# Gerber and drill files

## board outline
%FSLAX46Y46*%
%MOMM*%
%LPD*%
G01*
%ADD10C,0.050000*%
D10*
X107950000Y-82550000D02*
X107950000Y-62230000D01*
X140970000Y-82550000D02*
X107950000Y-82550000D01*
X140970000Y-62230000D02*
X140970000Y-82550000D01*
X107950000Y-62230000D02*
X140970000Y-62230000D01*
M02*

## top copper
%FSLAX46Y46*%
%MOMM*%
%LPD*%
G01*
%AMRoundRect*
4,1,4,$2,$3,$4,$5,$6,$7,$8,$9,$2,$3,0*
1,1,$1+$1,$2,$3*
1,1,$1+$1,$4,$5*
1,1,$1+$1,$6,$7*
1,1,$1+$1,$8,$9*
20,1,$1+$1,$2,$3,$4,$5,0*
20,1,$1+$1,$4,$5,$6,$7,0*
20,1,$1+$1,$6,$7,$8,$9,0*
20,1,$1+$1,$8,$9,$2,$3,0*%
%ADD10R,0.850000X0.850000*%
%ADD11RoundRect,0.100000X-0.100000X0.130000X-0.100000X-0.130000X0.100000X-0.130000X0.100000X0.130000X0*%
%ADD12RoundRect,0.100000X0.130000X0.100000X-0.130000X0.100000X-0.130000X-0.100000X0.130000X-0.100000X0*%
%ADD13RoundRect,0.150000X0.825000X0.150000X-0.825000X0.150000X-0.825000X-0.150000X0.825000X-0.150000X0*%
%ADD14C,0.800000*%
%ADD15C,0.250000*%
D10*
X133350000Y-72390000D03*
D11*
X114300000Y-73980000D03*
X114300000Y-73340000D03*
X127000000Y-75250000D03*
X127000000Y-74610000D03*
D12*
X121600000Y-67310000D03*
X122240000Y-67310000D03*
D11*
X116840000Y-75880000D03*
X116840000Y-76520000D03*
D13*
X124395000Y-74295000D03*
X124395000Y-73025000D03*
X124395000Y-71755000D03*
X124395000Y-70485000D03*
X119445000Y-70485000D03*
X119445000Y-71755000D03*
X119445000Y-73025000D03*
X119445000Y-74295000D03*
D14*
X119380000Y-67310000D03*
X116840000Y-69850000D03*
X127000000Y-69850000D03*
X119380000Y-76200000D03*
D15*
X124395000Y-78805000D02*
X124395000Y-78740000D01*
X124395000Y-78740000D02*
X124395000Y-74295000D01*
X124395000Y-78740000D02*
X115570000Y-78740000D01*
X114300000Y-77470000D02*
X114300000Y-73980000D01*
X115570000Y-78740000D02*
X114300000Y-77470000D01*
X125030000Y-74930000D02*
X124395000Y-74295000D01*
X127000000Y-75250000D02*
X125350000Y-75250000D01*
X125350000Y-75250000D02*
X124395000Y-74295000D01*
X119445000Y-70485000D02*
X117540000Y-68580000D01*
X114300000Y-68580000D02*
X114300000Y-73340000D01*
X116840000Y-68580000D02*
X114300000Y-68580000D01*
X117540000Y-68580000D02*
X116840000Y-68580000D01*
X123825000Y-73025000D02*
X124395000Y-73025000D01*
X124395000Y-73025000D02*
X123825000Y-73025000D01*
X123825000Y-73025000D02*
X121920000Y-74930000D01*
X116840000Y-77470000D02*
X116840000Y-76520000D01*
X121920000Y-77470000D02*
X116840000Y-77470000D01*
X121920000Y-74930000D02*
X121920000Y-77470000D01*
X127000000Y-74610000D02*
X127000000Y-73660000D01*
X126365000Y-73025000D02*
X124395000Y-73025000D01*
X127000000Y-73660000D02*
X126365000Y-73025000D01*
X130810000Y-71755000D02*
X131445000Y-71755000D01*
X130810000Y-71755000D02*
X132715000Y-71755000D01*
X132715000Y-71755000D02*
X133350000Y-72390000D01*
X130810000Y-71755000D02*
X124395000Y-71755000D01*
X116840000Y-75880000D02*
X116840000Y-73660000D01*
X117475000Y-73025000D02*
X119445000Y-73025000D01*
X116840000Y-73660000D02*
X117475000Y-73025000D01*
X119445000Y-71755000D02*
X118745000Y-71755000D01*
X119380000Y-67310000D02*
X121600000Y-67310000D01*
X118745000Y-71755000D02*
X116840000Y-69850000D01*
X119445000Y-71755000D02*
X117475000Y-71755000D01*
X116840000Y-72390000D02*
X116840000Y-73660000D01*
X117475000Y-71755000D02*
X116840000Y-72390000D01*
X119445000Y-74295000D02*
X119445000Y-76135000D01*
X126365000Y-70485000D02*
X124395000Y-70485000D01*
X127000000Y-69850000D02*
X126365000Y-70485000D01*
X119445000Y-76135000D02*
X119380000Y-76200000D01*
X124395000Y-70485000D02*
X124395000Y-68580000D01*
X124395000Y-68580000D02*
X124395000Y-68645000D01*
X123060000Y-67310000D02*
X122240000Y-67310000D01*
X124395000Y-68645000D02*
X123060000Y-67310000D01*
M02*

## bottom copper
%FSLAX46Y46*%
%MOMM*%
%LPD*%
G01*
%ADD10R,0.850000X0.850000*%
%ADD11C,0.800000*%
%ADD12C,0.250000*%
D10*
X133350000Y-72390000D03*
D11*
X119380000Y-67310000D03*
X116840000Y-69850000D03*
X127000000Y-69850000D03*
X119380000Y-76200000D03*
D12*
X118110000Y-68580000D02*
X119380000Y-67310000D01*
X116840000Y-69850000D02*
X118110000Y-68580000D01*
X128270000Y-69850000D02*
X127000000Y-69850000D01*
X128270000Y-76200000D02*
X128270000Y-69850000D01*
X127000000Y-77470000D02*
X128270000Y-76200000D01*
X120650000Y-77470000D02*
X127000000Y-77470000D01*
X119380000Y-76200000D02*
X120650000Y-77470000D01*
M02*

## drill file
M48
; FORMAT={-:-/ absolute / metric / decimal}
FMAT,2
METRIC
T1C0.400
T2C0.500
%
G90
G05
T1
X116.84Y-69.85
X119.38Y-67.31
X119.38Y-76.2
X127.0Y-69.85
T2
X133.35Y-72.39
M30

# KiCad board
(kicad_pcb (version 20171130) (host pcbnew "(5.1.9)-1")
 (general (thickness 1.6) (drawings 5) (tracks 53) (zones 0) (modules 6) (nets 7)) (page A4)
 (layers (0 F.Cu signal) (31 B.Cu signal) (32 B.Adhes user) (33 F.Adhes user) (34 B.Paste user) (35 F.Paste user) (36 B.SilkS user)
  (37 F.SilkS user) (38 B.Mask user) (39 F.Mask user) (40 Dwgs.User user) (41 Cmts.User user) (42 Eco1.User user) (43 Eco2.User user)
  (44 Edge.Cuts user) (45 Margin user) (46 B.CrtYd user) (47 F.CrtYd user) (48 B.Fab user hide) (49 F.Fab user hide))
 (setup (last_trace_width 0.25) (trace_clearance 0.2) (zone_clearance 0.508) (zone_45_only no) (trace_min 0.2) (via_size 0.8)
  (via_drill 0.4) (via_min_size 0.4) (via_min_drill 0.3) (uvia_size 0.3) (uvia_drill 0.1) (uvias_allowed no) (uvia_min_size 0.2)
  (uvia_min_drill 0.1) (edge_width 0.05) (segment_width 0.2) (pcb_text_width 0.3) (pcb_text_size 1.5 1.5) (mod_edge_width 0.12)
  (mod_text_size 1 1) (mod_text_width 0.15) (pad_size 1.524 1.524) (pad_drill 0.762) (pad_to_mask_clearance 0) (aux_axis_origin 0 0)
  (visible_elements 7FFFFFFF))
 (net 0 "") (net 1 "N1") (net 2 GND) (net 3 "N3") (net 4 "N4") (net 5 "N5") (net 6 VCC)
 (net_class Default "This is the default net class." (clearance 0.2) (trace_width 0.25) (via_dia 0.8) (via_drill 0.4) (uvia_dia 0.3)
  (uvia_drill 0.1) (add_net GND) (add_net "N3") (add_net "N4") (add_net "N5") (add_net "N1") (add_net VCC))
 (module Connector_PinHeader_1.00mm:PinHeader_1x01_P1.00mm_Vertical (layer F.Cu) (at 133.35 72.39)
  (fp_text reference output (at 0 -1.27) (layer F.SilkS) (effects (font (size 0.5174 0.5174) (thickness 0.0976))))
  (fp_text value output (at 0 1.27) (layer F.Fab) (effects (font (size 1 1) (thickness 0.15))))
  (pad 1 thru_hole rect (at 0 0) (size 0.85 0.85) (drill 0.5) (layers *.Cu *.Mask) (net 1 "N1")))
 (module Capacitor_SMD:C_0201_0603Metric (layer F.Cu) (at 114.3 73.66 270)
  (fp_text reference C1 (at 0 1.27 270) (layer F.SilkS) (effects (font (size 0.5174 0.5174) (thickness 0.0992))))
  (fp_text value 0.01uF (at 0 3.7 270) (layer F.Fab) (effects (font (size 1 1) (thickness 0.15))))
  (pad 2 smd roundrect (at 0.32 0 270) (size 0.46 0.4) (layers F.Cu F.Mask) (roundrect_rratio 0.25) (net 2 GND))
  (pad 1 smd roundrect (at -0.32 0 270) (size 0.46 0.4) (layers F.Cu F.Mask) (roundrect_rratio 0.25) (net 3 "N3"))
  (pad "" smd roundrect (at 0.345 0 270) (size 0.318 0.36) (layers F.Paste) (roundrect_rratio 0.25))
  (pad "" smd roundrect (at -0.345 0 270) (size 0.318 0.36) (layers F.Paste) (roundrect_rratio 0.25)))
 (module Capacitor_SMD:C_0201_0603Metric (layer F.Cu) (at 127 74.93 270)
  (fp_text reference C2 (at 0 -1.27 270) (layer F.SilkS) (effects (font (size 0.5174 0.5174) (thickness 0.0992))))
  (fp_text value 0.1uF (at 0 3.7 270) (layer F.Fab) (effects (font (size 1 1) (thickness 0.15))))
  (pad 2 smd roundrect (at 0.32 0 270) (size 0.46 0.4) (layers F.Cu F.Mask) (roundrect_rratio 0.25) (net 2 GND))
  (pad 1 smd roundrect (at -0.32 0 270) (size 0.46 0.4) (layers F.Cu F.Mask) (roundrect_rratio 0.25) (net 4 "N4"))
  (pad "" smd roundrect (at 0.345 0 270) (size 0.318 0.36) (layers F.Paste) (roundrect_rratio 0.25))
  (pad "" smd roundrect (at -0.345 0 270) (size 0.318 0.36) (layers F.Paste) (roundrect_rratio 0.25)))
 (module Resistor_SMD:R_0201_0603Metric (layer F.Cu) (at 121.92 67.31 180)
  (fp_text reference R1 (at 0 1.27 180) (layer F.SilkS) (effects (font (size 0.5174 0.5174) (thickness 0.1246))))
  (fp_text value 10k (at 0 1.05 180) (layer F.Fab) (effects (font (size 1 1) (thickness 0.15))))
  (pad 2 smd roundrect (at 0.32 0 180) (size 0.46 0.4) (layers F.Cu F.Mask) (roundrect_rratio 0.25) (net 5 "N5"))
  (pad 1 smd roundrect (at -0.32 0 180) (size 0.46 0.4) (layers F.Cu F.Mask) (roundrect_rratio 0.25) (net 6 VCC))
  (pad "" smd roundrect (at 0.345 0 180) (size 0.318 0.36) (layers F.Paste) (roundrect_rratio 0.25))
  (pad "" smd roundrect (at -0.345 0 180) (size 0.318 0.36) (layers F.Paste) (roundrect_rratio 0.25)))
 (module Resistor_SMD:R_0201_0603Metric (layer F.Cu) (at 116.84 76.2 270)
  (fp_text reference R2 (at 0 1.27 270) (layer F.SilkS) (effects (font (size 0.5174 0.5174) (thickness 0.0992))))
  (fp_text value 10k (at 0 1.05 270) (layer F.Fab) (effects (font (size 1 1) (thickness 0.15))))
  (pad "" smd roundrect (at -0.345 0 270) (size 0.318 0.36) (layers F.Paste) (roundrect_rratio 0.25))
  (pad "" smd roundrect (at 0.345 0 270) (size 0.318 0.36) (layers F.Paste) (roundrect_rratio 0.25))
  (pad 1 smd roundrect (at -0.32 0 270) (size 0.46 0.4) (layers F.Cu F.Mask) (roundrect_rratio 0.25) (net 5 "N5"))
  (pad 2 smd roundrect (at 0.32 0 270) (size 0.46 0.4) (layers F.Cu F.Mask) (roundrect_rratio 0.25) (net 4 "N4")))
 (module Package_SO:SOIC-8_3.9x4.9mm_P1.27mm (layer F.Cu) (at 121.92 72.39 180)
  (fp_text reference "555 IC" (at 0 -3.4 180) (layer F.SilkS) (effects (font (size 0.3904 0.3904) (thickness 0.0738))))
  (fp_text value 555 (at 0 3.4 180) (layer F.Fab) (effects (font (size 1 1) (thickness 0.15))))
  (pad 1 smd roundrect (at -2.475 -1.905 180) (size 1.95 0.6) (layers F.Cu F.Paste F.Mask) (roundrect_rratio 0.25) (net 2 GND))
  (pad 2 smd roundrect (at -2.475 -0.635 180) (size 1.95 0.6) (layers F.Cu F.Paste F.Mask) (roundrect_rratio 0.25) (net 4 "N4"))
  (pad 3 smd roundrect (at -2.475 0.635 180) (size 1.95 0.6) (layers F.Cu F.Paste F.Mask) (roundrect_rratio 0.25) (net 1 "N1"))
  (pad 4 smd roundrect (at -2.475 1.905 180) (size 1.95 0.6) (layers F.Cu F.Paste F.Mask) (roundrect_rratio 0.25) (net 6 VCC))
  (pad 5 smd roundrect (at 2.475 1.905 180) (size 1.95 0.6) (layers F.Cu F.Paste F.Mask) (roundrect_rratio 0.25) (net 3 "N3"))
  (pad 6 smd roundrect (at 2.475 0.635 180) (size 1.95 0.6) (layers F.Cu F.Paste F.Mask) (roundrect_rratio 0.25) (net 5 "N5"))
  (pad 7 smd roundrect (at 2.475 -0.635 180) (size 1.95 0.6) (layers F.Cu F.Paste F.Mask) (roundrect_rratio 0.25) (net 5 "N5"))
  (pad 8 smd roundrect (at 2.475 -1.905 180) (size 1.95 0.6) (layers F.Cu F.Paste F.Mask) (roundrect_rratio 0.25) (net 6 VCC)))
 (gr_line (start 107.95 82.55) (end 107.95 62.23) (angle 90) (layer Edge.Cuts) (width 0.05))
 (gr_line (start 140.97 82.55) (end 107.95 82.55) (angle 90) (layer Edge.Cuts) (width 0.05))
 (gr_line (start 140.97 62.23) (end 140.97 82.55) (angle 90) (layer Edge.Cuts) (width 0.05))
 (gr_line (start 107.95 62.23) (end 140.97 62.23) (angle 90) (layer Edge.Cuts) (width 0.05))
 (segment (start 124.395 78.805) (end 124.395 78.74) (width 0.25) (layer F.Cu) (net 2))
 (segment (start 124.395 78.74) (end 124.395 74.295) (width 0.25) (layer F.Cu) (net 2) (status 800000))
 (segment (start 124.395 78.74) (end 115.57 78.74) (width 0.25) (layer F.Cu) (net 2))
 (segment (start 114.3 77.47) (end 114.3 73.98) (width 0.25) (layer F.Cu) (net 2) (status 800000))
 (segment (start 115.57 78.74) (end 114.3 77.47) (width 0.25) (layer F.Cu) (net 2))
 (segment (start 125.03 74.93) (end 124.395 74.295) (width 0.25) (layer F.Cu) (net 2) (status 800000))
 (segment (start 127 75.25) (end 125.35 75.25) (width 0.25) (layer F.Cu) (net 2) (status 400000))
 (segment (start 125.35 75.25) (end 124.395 74.295) (width 0.25) (layer F.Cu) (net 2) (status 800000))
 (segment (start 119.445 70.485) (end 117.54 68.58) (width 0.25) (layer F.Cu) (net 3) (status 400000))
 (segment (start 114.3 68.58) (end 114.3 73.34) (width 0.25) (layer F.Cu) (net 3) (status 800000))
 (segment (start 116.84 68.58) (end 114.3 68.58) (width 0.25) (layer F.Cu) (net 3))
 (segment (start 117.54 68.58) (end 116.84 68.58) (width 0.25) (layer F.Cu) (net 3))
 (segment (start 123.825 73.025) (end 124.395 73.025) (width 0.25) (layer F.Cu) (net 4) (status C00000))
 (segment (start 124.395 73.025) (end 123.825 73.025) (width 0.25) (layer F.Cu) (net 4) (status C00000))
 (segment (start 123.825 73.025) (end 121.92 74.93) (width 0.25) (layer F.Cu) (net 4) (status 400000))
 (segment (start 116.84 77.47) (end 116.84 76.52) (width 0.25) (layer F.Cu) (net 4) (status 800000))
 (segment (start 121.92 77.47) (end 116.84 77.47) (width 0.25) (layer F.Cu) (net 4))
 (segment (start 121.92 74.93) (end 121.92 77.47) (width 0.25) (layer F.Cu) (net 4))
 (segment (start 127 74.61) (end 127 73.66) (width 0.25) (layer F.Cu) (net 4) (status 400000))
 (segment (start 126.365 73.025) (end 124.395 73.025) (width 0.25) (layer F.Cu) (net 4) (status 800000))
 (segment (start 127 73.66) (end 126.365 73.025) (width 0.25) (layer F.Cu) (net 4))
 (segment (start 130.81 71.755) (end 131.445 71.755) (width 0.25) (layer F.Cu) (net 1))
 (segment (start 130.81 71.755) (end 132.715 71.755) (width 0.25) (layer F.Cu) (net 1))
 (segment (start 132.715 71.755) (end 133.35 72.39) (width 0.25) (layer F.Cu) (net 1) (status 800000))
 (segment (start 130.81 71.755) (end 124.395 71.755) (width 0.25) (layer F.Cu) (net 1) (status 800000))
 (segment (start 116.84 75.88) (end 116.84 73.66) (width 0.25) (layer F.Cu) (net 5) (status 400000))
 (segment (start 117.475 73.025) (end 119.445 73.025) (width 0.25) (layer F.Cu) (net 5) (status 800000))
 (segment (start 116.84 73.66) (end 117.475 73.025) (width 0.25) (layer F.Cu) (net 5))
 (segment (start 119.445 71.755) (end 118.745 71.755) (width 0.25) (layer F.Cu) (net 5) (status C00000))
 (segment (start 119.38 67.31) (end 121.6 67.31) (width 0.25) (layer F.Cu) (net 5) (status 800000))
 (via (at 119.38 67.31) (size 0.8) (drill 0.4) (layers F.Cu B.Cu) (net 5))
 (segment (start 118.11 68.58) (end 119.38 67.31) (width 0.25) (layer B.Cu) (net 5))
 (segment (start 118.745 71.755) (end 116.84 69.85) (width 0.25) (layer F.Cu) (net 5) (status 400000))
 (via (at 116.84 69.85) (size 0.8) (drill 0.4) (layers F.Cu B.Cu) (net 5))
 (segment (start 116.84 69.85) (end 118.11 68.58) (width 0.25) (layer B.Cu) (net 5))
 (segment (start 119.445 71.755) (end 117.475 71.755) (width 0.25) (layer F.Cu) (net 5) (status 400000))
 (segment (start 116.84 72.39) (end 116.84 73.66) (width 0.25) (layer F.Cu) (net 5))
 (segment (start 117.475 71.755) (end 116.84 72.39) (width 0.25) (layer F.Cu) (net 5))
 (segment (start 119.445 74.295) (end 119.445 76.135) (width 0.25) (layer F.Cu) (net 6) (status 400000))
 (segment (start 126.365 70.485) (end 124.395 70.485) (width 0.25) (layer F.Cu) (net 6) (status 800000))
 (segment (start 127 69.85) (end 126.365 70.485) (width 0.25) (layer F.Cu) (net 6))
 (via (at 127 69.85) (size 0.8) (drill 0.4) (layers F.Cu B.Cu) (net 6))
 (segment (start 128.27 69.85) (end 127 69.85) (width 0.25) (layer B.Cu) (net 6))
 (segment (start 128.27 76.2) (end 128.27 69.85) (width 0.25) (layer B.Cu) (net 6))
 (segment (start 127 77.47) (end 128.27 76.2) (width 0.25) (layer B.Cu) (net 6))
 (segment (start 120.65 77.47) (end 127 77.47) (width 0.25) (layer B.Cu) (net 6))
 (segment (start 119.38 76.2) (end 120.65 77.47) (width 0.25) (layer B.Cu) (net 6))
 (via (at 119.38 76.2) (size 0.8) (drill 0.4) (layers F.Cu B.Cu) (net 6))
 (segment (start 119.445 76.135) (end 119.38 76.2) (width 0.25) (layer F.Cu) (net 6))
 (segment (start 124.395 70.485) (end 124.395 68.58) (width 0.25) (layer F.Cu) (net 6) (status 400000))
 (segment (start 124.395 68.58) (end 124.395 68.645) (width 0.25) (layer F.Cu) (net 6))
 (segment (start 123.06 67.31) (end 122.24 67.31) (width 0.25) (layer F.Cu) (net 6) (status 800000))
 (segment (start 124.395 68.645) (end 123.06 67.31) (width 0.25) (layer F.Cu) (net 6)))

